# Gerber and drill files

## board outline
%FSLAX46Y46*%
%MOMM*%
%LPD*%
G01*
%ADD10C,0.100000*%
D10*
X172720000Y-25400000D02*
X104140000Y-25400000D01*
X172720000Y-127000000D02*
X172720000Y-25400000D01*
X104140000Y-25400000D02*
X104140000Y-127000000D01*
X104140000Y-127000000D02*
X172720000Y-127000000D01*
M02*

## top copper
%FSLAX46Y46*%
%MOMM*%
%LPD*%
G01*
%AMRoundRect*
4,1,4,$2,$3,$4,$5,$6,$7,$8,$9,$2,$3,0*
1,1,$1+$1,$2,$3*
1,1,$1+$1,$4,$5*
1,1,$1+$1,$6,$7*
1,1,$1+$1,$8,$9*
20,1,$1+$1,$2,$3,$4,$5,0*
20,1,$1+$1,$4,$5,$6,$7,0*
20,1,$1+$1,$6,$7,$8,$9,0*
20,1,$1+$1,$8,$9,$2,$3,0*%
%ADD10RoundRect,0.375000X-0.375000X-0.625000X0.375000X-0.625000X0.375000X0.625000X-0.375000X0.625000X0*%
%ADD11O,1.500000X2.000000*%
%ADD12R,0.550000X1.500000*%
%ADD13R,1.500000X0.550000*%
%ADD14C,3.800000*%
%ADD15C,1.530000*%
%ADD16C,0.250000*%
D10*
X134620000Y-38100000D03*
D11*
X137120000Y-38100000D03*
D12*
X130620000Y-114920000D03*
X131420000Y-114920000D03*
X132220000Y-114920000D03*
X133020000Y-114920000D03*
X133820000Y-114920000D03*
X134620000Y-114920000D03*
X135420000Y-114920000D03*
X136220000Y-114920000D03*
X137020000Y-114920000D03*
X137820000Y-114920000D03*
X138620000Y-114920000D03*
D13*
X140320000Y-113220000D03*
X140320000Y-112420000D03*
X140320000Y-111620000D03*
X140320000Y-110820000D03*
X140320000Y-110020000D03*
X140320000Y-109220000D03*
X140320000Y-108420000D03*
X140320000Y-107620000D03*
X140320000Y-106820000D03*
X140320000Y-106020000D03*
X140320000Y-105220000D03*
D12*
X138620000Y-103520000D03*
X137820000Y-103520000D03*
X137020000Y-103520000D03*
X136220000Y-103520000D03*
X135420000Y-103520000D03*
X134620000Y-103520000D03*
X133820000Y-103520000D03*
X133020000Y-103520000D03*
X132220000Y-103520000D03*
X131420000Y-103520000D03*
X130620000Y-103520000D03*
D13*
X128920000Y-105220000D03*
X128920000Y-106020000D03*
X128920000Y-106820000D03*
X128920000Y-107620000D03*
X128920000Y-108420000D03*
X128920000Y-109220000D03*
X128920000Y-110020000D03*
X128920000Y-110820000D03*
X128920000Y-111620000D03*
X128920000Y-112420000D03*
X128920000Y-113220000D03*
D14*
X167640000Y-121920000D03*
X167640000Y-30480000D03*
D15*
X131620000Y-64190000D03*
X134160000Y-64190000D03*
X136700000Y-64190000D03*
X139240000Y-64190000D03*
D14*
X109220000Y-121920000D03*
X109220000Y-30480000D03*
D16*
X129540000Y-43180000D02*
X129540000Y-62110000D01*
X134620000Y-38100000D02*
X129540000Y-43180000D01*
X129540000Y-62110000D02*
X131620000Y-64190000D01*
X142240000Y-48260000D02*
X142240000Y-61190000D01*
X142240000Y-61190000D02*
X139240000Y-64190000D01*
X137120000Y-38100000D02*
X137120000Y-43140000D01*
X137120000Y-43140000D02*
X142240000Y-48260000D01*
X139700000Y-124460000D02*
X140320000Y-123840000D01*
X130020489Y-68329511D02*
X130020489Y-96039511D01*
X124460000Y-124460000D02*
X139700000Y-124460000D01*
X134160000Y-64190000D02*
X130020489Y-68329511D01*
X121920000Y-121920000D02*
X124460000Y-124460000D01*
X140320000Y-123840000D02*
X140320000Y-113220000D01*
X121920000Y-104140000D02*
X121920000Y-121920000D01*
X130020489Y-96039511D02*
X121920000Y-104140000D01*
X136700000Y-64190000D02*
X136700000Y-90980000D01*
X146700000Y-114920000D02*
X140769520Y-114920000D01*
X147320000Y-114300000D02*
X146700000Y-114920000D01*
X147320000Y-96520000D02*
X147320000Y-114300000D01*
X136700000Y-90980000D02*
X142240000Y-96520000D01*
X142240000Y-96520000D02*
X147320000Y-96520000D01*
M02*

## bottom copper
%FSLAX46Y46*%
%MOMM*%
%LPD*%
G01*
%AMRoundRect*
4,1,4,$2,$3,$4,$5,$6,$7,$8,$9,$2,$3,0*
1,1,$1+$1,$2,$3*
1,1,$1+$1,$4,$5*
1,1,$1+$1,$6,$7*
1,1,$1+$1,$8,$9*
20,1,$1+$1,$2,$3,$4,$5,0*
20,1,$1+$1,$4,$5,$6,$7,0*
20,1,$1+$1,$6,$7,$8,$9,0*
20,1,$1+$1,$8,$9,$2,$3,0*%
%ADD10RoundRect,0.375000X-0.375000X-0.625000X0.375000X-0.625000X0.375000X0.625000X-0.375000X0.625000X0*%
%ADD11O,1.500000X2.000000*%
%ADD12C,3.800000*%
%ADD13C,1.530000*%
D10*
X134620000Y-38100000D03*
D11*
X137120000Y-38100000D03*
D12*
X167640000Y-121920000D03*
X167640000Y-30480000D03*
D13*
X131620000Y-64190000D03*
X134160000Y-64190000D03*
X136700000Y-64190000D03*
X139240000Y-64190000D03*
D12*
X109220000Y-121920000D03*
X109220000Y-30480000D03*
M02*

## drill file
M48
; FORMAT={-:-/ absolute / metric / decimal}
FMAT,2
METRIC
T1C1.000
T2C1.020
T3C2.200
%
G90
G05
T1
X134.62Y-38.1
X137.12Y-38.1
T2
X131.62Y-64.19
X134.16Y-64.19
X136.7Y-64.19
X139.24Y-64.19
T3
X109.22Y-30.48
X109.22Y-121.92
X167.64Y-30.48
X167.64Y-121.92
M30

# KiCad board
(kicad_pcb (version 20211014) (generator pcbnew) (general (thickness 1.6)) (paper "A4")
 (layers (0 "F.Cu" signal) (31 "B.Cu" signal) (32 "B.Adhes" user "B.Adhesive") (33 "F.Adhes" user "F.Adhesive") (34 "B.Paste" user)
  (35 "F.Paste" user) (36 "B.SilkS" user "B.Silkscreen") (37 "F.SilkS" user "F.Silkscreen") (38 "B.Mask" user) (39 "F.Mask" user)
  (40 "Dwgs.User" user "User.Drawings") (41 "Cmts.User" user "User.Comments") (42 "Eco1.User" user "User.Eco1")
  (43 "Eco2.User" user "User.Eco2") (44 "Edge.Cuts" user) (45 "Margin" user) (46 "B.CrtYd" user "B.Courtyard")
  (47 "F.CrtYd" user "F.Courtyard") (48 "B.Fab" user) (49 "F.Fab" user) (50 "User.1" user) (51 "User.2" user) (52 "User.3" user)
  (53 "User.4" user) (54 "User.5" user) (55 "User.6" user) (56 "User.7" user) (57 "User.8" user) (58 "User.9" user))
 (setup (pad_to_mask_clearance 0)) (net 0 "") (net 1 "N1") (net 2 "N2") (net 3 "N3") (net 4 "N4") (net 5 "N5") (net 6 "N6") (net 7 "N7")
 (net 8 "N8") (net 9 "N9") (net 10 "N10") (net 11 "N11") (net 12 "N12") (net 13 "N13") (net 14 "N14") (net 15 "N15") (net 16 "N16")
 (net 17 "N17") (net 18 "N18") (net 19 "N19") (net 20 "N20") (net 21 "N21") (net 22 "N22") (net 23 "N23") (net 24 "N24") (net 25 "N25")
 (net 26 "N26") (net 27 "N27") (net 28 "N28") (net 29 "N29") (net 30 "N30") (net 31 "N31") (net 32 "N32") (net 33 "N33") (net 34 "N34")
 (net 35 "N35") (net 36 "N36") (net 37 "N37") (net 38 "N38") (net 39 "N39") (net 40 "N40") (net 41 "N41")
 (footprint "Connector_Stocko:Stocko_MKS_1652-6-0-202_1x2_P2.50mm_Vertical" (layer "F.Cu") (at 134.62 38.1)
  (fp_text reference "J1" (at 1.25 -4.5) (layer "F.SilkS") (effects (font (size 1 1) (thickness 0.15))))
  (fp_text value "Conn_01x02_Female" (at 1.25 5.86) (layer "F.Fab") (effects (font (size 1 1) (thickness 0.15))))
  (pad "1" thru_hole roundrect (at 0 0) (size 1.5 2) (drill 1) (layers *.Cu *.Mask) (roundrect_rratio 0.25) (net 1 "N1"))
  (pad "2" thru_hole oval (at 2.5 0) (size 1.5 2) (drill 1) (layers *.Cu *.Mask) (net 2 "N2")))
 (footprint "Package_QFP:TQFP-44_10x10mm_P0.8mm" (layer "F.Cu") (at 134.62 109.22 90)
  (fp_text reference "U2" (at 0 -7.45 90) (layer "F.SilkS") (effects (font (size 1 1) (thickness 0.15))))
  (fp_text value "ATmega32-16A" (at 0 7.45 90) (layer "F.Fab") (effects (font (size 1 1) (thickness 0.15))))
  (pad "1" smd rect (at -5.7 -4 90) (size 1.5 0.55) (layers "F.Cu" "F.Paste" "F.Mask") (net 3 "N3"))
  (pad "2" smd rect (at -5.7 -3.2 90) (size 1.5 0.55) (layers "F.Cu" "F.Paste" "F.Mask") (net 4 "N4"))
  (pad "3" smd rect (at -5.7 -2.4 90) (size 1.5 0.55) (layers "F.Cu" "F.Paste" "F.Mask") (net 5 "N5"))
  (pad "4" smd rect (at -5.7 -1.6 90) (size 1.5 0.55) (layers "F.Cu" "F.Paste" "F.Mask") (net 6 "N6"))
  (pad "5" smd rect (at -5.7 -0.8 90) (size 1.5 0.55) (layers "F.Cu" "F.Paste" "F.Mask") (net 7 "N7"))
  (pad "6" smd rect (at -5.7 0 90) (size 1.5 0.55) (layers "F.Cu" "F.Paste" "F.Mask") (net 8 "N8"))
  (pad "7" smd rect (at -5.7 0.8 90) (size 1.5 0.55) (layers "F.Cu" "F.Paste" "F.Mask") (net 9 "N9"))
  (pad "8" smd rect (at -5.7 1.6 90) (size 1.5 0.55) (layers "F.Cu" "F.Paste" "F.Mask") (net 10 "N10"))
  (pad "9" smd rect (at -5.7 2.4 90) (size 1.5 0.55) (layers "F.Cu" "F.Paste" "F.Mask") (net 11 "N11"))
  (pad "10" smd rect (at -5.7 3.2 90) (size 1.5 0.55) (layers "F.Cu" "F.Paste" "F.Mask") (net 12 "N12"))
  (pad "11" smd rect (at -5.7 4 90) (size 1.5 0.55) (layers "F.Cu" "F.Paste" "F.Mask") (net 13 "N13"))
  (pad "12" smd rect (at -4 5.7 180) (size 1.5 0.55) (layers "F.Cu" "F.Paste" "F.Mask") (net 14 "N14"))
  (pad "13" smd rect (at -3.2 5.7 180) (size 1.5 0.55) (layers "F.Cu" "F.Paste" "F.Mask") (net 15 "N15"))
  (pad "14" smd rect (at -2.4 5.7 180) (size 1.5 0.55) (layers "F.Cu" "F.Paste" "F.Mask") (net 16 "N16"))
  (pad "15" smd rect (at -1.6 5.7 180) (size 1.5 0.55) (layers "F.Cu" "F.Paste" "F.Mask") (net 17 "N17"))
  (pad "16" smd rect (at -0.8 5.7 180) (size 1.5 0.55) (layers "F.Cu" "F.Paste" "F.Mask") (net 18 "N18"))
  (pad "17" smd rect (at 0 5.7 180) (size 1.5 0.55) (layers "F.Cu" "F.Paste" "F.Mask") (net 7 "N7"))
  (pad "18" smd rect (at 0.8 5.7 180) (size 1.5 0.55) (layers "F.Cu" "F.Paste" "F.Mask") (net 8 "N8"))
  (pad "19" smd rect (at 1.6 5.7 180) (size 1.5 0.55) (layers "F.Cu" "F.Paste" "F.Mask") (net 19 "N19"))
  (pad "20" smd rect (at 2.4 5.7 180) (size 1.5 0.55) (layers "F.Cu" "F.Paste" "F.Mask") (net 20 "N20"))
  (pad "21" smd rect (at 3.2 5.7 180) (size 1.5 0.55) (layers "F.Cu" "F.Paste" "F.Mask") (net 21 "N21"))
  (pad "22" smd rect (at 4 5.7 180) (size 1.5 0.55) (layers "F.Cu" "F.Paste" "F.Mask") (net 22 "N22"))
  (pad "23" smd rect (at 5.7 4 90) (size 1.5 0.55) (layers "F.Cu" "F.Paste" "F.Mask") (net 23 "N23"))
  (pad "24" smd rect (at 5.7 3.2 90) (size 1.5 0.55) (layers "F.Cu" "F.Paste" "F.Mask") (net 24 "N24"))
  (pad "25" smd rect (at 5.7 2.4 90) (size 1.5 0.55) (layers "F.Cu" "F.Paste" "F.Mask") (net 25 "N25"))
  (pad "26" smd rect (at 5.7 1.6 90) (size 1.5 0.55) (layers "F.Cu" "F.Paste" "F.Mask") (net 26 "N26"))
  (pad "27" smd rect (at 5.7 0.8 90) (size 1.5 0.55) (layers "F.Cu" "F.Paste" "F.Mask") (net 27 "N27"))
  (pad "28" smd rect (at 5.7 0 90) (size 1.5 0.55) (layers "F.Cu" "F.Paste" "F.Mask") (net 8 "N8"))
  (pad "29" smd rect (at 5.7 -0.8 90) (size 1.5 0.55) (layers "F.Cu" "F.Paste" "F.Mask") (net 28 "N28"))
  (pad "30" smd rect (at 5.7 -1.6 90) (size 1.5 0.55) (layers "F.Cu" "F.Paste" "F.Mask") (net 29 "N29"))
  (pad "31" smd rect (at 5.7 -2.4 90) (size 1.5 0.55) (layers "F.Cu" "F.Paste" "F.Mask") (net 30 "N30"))
  (pad "32" smd rect (at 5.7 -3.2 90) (size 1.5 0.55) (layers "F.Cu" "F.Paste" "F.Mask") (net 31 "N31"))
  (pad "33" smd rect (at 5.7 -4 90) (size 1.5 0.55) (layers "F.Cu" "F.Paste" "F.Mask") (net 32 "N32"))
  (pad "34" smd rect (at 4 -5.7 180) (size 1.5 0.55) (layers "F.Cu" "F.Paste" "F.Mask") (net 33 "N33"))
  (pad "35" smd rect (at 3.2 -5.7 180) (size 1.5 0.55) (layers "F.Cu" "F.Paste" "F.Mask") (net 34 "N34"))
  (pad "36" smd rect (at 2.4 -5.7 180) (size 1.5 0.55) (layers "F.Cu" "F.Paste" "F.Mask") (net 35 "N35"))
  (pad "37" smd rect (at 1.6 -5.7 180) (size 1.5 0.55) (layers "F.Cu" "F.Paste" "F.Mask") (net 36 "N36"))
  (pad "38" smd rect (at 0.8 -5.7 180) (size 1.5 0.55) (layers "F.Cu" "F.Paste" "F.Mask") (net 7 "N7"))
  (pad "39" smd rect (at 0 -5.7 180) (size 1.5 0.55) (layers "F.Cu" "F.Paste" "F.Mask") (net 8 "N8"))
  (pad "40" smd rect (at -0.8 -5.7 180) (size 1.5 0.55) (layers "F.Cu" "F.Paste" "F.Mask") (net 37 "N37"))
  (pad "41" smd rect (at -1.6 -5.7 180) (size 1.5 0.55) (layers "F.Cu" "F.Paste" "F.Mask") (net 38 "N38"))
  (pad "42" smd rect (at -2.4 -5.7 180) (size 1.5 0.55) (layers "F.Cu" "F.Paste" "F.Mask") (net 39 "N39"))
  (pad "43" smd rect (at -3.2 -5.7 180) (size 1.5 0.55) (layers "F.Cu" "F.Paste" "F.Mask") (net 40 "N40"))
  (pad "44" smd rect (at -4 -5.7 180) (size 1.5 0.55) (layers "F.Cu" "F.Paste" "F.Mask") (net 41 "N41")))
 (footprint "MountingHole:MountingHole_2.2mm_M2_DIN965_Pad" (layer "F.Cu") (at 167.64 121.92)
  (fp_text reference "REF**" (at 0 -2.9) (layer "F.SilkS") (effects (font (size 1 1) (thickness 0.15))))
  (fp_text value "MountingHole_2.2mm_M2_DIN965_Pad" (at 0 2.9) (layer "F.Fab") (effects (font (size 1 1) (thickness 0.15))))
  (pad "1" thru_hole circle (at 0 0) (size 3.8 3.8) (drill 2.2) (layers *.Cu *.Mask)))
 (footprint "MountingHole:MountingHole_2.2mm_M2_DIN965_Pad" (layer "F.Cu") (at 167.64 30.48)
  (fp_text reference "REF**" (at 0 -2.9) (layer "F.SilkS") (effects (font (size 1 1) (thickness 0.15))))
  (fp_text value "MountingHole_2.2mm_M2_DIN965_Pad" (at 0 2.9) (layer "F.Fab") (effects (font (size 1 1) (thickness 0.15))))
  (pad "1" thru_hole circle (at 0 0) (size 3.8 3.8) (drill 2.2) (layers *.Cu *.Mask)))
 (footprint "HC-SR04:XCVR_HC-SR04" (layer "F.Cu") (at 135.43 64.19)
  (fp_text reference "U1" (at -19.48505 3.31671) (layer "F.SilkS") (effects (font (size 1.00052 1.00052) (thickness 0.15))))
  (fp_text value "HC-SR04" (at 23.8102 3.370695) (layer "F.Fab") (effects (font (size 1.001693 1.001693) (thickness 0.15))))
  (pad "1" thru_hole circle locked (at -3.81 0) (size 1.53 1.53) (drill 1.02) (layers *.Cu *.Mask) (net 1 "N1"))
  (pad "2" thru_hole circle locked (at -1.27 0) (size 1.53 1.53) (drill 1.02) (layers *.Cu *.Mask) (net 14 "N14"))
  (pad "3" thru_hole circle locked (at 1.27 0) (size 1.53 1.53) (drill 1.02) (layers *.Cu *.Mask) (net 13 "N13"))
  (pad "4" thru_hole circle locked (at 3.81 0) (size 1.53 1.53) (drill 1.02) (layers *.Cu *.Mask) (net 2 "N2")))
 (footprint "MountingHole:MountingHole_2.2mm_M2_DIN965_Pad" (layer "F.Cu") (at 109.22 121.92)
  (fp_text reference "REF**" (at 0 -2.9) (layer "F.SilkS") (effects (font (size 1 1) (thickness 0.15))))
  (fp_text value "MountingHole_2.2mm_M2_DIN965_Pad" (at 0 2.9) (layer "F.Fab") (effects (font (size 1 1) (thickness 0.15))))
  (pad "1" thru_hole circle (at 0 0) (size 3.8 3.8) (drill 2.2) (layers *.Cu *.Mask)))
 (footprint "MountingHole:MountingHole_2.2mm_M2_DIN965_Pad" (layer "F.Cu") (at 109.22 30.48)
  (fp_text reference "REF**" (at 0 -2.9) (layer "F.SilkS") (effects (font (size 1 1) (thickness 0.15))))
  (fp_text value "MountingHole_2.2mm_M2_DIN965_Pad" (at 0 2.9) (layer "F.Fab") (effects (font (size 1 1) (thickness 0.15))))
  (pad "1" thru_hole circle (at 0 0) (size 3.8 3.8) (drill 2.2) (layers *.Cu *.Mask)))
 (gr_line (start 172.72 25.4) (end 104.14 25.4) (layer "Edge.Cuts") (width 0.1))
 (gr_line (start 172.72 127) (end 172.72 25.4) (layer "Edge.Cuts") (width 0.1))
 (gr_line (start 104.14 25.4) (end 104.14 127) (layer "Edge.Cuts") (width 0.1))
 (gr_line (start 104.14 127) (end 172.72 127) (layer "Edge.Cuts") (width 0.1))
 (segment (start 129.54 43.18) (end 129.54 62.11) (width 0.25) (layer "F.Cu") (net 1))
 (segment (start 134.62 38.1) (end 129.54 43.18) (width 0.25) (layer "F.Cu") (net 1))
 (segment (start 129.54 62.11) (end 131.62 64.19) (width 0.25) (layer "F.Cu") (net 1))
 (segment (start 142.24 48.26) (end 142.24 61.19) (width 0.25) (layer "F.Cu") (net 2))
 (segment (start 142.24 61.19) (end 139.24 64.19) (width 0.25) (layer "F.Cu") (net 2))
 (segment (start 137.12 38.1) (end 137.12 43.14) (width 0.25) (layer "F.Cu") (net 2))
 (segment (start 137.12 43.14) (end 142.24 48.26) (width 0.25) (layer "F.Cu") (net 2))
 (segment (start 139.7 124.46) (end 140.32 123.84) (width 0.25) (layer "F.Cu") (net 14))
 (segment (start 130.020489 68.329511) (end 130.020489 96.039511) (width 0.25) (layer "F.Cu") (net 14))
 (segment (start 124.46 124.46) (end 139.7 124.46) (width 0.25) (layer "F.Cu") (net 14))
 (segment (start 134.16 64.19) (end 130.020489 68.329511) (width 0.25) (layer "F.Cu") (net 14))
 (segment (start 121.92 121.92) (end 124.46 124.46) (width 0.25) (layer "F.Cu") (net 14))
 (segment (start 140.32 123.84) (end 140.32 113.22) (width 0.25) (layer "F.Cu") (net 14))
 (segment (start 121.92 104.14) (end 121.92 121.92) (width 0.25) (layer "F.Cu") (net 14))
 (segment (start 130.020489 96.039511) (end 121.92 104.14) (width 0.25) (layer "F.Cu") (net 14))
 (segment (start 136.7 64.19) (end 136.7 90.98) (width 0.25) (layer "F.Cu") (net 13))
 (segment (start 146.7 114.92) (end 140.76952 114.92) (width 0.25) (layer "F.Cu") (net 13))
 (segment (start 147.32 114.3) (end 146.7 114.92) (width 0.25) (layer "F.Cu") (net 13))
 (segment (start 147.32 96.52) (end 147.32 114.3) (width 0.25) (layer "F.Cu") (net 13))
 (segment (start 136.7 90.98) (end 142.24 96.52) (width 0.25) (layer "F.Cu") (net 13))
 (segment (start 142.24 96.52) (end 147.32 96.52) (width 0.25) (layer "F.Cu") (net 13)))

